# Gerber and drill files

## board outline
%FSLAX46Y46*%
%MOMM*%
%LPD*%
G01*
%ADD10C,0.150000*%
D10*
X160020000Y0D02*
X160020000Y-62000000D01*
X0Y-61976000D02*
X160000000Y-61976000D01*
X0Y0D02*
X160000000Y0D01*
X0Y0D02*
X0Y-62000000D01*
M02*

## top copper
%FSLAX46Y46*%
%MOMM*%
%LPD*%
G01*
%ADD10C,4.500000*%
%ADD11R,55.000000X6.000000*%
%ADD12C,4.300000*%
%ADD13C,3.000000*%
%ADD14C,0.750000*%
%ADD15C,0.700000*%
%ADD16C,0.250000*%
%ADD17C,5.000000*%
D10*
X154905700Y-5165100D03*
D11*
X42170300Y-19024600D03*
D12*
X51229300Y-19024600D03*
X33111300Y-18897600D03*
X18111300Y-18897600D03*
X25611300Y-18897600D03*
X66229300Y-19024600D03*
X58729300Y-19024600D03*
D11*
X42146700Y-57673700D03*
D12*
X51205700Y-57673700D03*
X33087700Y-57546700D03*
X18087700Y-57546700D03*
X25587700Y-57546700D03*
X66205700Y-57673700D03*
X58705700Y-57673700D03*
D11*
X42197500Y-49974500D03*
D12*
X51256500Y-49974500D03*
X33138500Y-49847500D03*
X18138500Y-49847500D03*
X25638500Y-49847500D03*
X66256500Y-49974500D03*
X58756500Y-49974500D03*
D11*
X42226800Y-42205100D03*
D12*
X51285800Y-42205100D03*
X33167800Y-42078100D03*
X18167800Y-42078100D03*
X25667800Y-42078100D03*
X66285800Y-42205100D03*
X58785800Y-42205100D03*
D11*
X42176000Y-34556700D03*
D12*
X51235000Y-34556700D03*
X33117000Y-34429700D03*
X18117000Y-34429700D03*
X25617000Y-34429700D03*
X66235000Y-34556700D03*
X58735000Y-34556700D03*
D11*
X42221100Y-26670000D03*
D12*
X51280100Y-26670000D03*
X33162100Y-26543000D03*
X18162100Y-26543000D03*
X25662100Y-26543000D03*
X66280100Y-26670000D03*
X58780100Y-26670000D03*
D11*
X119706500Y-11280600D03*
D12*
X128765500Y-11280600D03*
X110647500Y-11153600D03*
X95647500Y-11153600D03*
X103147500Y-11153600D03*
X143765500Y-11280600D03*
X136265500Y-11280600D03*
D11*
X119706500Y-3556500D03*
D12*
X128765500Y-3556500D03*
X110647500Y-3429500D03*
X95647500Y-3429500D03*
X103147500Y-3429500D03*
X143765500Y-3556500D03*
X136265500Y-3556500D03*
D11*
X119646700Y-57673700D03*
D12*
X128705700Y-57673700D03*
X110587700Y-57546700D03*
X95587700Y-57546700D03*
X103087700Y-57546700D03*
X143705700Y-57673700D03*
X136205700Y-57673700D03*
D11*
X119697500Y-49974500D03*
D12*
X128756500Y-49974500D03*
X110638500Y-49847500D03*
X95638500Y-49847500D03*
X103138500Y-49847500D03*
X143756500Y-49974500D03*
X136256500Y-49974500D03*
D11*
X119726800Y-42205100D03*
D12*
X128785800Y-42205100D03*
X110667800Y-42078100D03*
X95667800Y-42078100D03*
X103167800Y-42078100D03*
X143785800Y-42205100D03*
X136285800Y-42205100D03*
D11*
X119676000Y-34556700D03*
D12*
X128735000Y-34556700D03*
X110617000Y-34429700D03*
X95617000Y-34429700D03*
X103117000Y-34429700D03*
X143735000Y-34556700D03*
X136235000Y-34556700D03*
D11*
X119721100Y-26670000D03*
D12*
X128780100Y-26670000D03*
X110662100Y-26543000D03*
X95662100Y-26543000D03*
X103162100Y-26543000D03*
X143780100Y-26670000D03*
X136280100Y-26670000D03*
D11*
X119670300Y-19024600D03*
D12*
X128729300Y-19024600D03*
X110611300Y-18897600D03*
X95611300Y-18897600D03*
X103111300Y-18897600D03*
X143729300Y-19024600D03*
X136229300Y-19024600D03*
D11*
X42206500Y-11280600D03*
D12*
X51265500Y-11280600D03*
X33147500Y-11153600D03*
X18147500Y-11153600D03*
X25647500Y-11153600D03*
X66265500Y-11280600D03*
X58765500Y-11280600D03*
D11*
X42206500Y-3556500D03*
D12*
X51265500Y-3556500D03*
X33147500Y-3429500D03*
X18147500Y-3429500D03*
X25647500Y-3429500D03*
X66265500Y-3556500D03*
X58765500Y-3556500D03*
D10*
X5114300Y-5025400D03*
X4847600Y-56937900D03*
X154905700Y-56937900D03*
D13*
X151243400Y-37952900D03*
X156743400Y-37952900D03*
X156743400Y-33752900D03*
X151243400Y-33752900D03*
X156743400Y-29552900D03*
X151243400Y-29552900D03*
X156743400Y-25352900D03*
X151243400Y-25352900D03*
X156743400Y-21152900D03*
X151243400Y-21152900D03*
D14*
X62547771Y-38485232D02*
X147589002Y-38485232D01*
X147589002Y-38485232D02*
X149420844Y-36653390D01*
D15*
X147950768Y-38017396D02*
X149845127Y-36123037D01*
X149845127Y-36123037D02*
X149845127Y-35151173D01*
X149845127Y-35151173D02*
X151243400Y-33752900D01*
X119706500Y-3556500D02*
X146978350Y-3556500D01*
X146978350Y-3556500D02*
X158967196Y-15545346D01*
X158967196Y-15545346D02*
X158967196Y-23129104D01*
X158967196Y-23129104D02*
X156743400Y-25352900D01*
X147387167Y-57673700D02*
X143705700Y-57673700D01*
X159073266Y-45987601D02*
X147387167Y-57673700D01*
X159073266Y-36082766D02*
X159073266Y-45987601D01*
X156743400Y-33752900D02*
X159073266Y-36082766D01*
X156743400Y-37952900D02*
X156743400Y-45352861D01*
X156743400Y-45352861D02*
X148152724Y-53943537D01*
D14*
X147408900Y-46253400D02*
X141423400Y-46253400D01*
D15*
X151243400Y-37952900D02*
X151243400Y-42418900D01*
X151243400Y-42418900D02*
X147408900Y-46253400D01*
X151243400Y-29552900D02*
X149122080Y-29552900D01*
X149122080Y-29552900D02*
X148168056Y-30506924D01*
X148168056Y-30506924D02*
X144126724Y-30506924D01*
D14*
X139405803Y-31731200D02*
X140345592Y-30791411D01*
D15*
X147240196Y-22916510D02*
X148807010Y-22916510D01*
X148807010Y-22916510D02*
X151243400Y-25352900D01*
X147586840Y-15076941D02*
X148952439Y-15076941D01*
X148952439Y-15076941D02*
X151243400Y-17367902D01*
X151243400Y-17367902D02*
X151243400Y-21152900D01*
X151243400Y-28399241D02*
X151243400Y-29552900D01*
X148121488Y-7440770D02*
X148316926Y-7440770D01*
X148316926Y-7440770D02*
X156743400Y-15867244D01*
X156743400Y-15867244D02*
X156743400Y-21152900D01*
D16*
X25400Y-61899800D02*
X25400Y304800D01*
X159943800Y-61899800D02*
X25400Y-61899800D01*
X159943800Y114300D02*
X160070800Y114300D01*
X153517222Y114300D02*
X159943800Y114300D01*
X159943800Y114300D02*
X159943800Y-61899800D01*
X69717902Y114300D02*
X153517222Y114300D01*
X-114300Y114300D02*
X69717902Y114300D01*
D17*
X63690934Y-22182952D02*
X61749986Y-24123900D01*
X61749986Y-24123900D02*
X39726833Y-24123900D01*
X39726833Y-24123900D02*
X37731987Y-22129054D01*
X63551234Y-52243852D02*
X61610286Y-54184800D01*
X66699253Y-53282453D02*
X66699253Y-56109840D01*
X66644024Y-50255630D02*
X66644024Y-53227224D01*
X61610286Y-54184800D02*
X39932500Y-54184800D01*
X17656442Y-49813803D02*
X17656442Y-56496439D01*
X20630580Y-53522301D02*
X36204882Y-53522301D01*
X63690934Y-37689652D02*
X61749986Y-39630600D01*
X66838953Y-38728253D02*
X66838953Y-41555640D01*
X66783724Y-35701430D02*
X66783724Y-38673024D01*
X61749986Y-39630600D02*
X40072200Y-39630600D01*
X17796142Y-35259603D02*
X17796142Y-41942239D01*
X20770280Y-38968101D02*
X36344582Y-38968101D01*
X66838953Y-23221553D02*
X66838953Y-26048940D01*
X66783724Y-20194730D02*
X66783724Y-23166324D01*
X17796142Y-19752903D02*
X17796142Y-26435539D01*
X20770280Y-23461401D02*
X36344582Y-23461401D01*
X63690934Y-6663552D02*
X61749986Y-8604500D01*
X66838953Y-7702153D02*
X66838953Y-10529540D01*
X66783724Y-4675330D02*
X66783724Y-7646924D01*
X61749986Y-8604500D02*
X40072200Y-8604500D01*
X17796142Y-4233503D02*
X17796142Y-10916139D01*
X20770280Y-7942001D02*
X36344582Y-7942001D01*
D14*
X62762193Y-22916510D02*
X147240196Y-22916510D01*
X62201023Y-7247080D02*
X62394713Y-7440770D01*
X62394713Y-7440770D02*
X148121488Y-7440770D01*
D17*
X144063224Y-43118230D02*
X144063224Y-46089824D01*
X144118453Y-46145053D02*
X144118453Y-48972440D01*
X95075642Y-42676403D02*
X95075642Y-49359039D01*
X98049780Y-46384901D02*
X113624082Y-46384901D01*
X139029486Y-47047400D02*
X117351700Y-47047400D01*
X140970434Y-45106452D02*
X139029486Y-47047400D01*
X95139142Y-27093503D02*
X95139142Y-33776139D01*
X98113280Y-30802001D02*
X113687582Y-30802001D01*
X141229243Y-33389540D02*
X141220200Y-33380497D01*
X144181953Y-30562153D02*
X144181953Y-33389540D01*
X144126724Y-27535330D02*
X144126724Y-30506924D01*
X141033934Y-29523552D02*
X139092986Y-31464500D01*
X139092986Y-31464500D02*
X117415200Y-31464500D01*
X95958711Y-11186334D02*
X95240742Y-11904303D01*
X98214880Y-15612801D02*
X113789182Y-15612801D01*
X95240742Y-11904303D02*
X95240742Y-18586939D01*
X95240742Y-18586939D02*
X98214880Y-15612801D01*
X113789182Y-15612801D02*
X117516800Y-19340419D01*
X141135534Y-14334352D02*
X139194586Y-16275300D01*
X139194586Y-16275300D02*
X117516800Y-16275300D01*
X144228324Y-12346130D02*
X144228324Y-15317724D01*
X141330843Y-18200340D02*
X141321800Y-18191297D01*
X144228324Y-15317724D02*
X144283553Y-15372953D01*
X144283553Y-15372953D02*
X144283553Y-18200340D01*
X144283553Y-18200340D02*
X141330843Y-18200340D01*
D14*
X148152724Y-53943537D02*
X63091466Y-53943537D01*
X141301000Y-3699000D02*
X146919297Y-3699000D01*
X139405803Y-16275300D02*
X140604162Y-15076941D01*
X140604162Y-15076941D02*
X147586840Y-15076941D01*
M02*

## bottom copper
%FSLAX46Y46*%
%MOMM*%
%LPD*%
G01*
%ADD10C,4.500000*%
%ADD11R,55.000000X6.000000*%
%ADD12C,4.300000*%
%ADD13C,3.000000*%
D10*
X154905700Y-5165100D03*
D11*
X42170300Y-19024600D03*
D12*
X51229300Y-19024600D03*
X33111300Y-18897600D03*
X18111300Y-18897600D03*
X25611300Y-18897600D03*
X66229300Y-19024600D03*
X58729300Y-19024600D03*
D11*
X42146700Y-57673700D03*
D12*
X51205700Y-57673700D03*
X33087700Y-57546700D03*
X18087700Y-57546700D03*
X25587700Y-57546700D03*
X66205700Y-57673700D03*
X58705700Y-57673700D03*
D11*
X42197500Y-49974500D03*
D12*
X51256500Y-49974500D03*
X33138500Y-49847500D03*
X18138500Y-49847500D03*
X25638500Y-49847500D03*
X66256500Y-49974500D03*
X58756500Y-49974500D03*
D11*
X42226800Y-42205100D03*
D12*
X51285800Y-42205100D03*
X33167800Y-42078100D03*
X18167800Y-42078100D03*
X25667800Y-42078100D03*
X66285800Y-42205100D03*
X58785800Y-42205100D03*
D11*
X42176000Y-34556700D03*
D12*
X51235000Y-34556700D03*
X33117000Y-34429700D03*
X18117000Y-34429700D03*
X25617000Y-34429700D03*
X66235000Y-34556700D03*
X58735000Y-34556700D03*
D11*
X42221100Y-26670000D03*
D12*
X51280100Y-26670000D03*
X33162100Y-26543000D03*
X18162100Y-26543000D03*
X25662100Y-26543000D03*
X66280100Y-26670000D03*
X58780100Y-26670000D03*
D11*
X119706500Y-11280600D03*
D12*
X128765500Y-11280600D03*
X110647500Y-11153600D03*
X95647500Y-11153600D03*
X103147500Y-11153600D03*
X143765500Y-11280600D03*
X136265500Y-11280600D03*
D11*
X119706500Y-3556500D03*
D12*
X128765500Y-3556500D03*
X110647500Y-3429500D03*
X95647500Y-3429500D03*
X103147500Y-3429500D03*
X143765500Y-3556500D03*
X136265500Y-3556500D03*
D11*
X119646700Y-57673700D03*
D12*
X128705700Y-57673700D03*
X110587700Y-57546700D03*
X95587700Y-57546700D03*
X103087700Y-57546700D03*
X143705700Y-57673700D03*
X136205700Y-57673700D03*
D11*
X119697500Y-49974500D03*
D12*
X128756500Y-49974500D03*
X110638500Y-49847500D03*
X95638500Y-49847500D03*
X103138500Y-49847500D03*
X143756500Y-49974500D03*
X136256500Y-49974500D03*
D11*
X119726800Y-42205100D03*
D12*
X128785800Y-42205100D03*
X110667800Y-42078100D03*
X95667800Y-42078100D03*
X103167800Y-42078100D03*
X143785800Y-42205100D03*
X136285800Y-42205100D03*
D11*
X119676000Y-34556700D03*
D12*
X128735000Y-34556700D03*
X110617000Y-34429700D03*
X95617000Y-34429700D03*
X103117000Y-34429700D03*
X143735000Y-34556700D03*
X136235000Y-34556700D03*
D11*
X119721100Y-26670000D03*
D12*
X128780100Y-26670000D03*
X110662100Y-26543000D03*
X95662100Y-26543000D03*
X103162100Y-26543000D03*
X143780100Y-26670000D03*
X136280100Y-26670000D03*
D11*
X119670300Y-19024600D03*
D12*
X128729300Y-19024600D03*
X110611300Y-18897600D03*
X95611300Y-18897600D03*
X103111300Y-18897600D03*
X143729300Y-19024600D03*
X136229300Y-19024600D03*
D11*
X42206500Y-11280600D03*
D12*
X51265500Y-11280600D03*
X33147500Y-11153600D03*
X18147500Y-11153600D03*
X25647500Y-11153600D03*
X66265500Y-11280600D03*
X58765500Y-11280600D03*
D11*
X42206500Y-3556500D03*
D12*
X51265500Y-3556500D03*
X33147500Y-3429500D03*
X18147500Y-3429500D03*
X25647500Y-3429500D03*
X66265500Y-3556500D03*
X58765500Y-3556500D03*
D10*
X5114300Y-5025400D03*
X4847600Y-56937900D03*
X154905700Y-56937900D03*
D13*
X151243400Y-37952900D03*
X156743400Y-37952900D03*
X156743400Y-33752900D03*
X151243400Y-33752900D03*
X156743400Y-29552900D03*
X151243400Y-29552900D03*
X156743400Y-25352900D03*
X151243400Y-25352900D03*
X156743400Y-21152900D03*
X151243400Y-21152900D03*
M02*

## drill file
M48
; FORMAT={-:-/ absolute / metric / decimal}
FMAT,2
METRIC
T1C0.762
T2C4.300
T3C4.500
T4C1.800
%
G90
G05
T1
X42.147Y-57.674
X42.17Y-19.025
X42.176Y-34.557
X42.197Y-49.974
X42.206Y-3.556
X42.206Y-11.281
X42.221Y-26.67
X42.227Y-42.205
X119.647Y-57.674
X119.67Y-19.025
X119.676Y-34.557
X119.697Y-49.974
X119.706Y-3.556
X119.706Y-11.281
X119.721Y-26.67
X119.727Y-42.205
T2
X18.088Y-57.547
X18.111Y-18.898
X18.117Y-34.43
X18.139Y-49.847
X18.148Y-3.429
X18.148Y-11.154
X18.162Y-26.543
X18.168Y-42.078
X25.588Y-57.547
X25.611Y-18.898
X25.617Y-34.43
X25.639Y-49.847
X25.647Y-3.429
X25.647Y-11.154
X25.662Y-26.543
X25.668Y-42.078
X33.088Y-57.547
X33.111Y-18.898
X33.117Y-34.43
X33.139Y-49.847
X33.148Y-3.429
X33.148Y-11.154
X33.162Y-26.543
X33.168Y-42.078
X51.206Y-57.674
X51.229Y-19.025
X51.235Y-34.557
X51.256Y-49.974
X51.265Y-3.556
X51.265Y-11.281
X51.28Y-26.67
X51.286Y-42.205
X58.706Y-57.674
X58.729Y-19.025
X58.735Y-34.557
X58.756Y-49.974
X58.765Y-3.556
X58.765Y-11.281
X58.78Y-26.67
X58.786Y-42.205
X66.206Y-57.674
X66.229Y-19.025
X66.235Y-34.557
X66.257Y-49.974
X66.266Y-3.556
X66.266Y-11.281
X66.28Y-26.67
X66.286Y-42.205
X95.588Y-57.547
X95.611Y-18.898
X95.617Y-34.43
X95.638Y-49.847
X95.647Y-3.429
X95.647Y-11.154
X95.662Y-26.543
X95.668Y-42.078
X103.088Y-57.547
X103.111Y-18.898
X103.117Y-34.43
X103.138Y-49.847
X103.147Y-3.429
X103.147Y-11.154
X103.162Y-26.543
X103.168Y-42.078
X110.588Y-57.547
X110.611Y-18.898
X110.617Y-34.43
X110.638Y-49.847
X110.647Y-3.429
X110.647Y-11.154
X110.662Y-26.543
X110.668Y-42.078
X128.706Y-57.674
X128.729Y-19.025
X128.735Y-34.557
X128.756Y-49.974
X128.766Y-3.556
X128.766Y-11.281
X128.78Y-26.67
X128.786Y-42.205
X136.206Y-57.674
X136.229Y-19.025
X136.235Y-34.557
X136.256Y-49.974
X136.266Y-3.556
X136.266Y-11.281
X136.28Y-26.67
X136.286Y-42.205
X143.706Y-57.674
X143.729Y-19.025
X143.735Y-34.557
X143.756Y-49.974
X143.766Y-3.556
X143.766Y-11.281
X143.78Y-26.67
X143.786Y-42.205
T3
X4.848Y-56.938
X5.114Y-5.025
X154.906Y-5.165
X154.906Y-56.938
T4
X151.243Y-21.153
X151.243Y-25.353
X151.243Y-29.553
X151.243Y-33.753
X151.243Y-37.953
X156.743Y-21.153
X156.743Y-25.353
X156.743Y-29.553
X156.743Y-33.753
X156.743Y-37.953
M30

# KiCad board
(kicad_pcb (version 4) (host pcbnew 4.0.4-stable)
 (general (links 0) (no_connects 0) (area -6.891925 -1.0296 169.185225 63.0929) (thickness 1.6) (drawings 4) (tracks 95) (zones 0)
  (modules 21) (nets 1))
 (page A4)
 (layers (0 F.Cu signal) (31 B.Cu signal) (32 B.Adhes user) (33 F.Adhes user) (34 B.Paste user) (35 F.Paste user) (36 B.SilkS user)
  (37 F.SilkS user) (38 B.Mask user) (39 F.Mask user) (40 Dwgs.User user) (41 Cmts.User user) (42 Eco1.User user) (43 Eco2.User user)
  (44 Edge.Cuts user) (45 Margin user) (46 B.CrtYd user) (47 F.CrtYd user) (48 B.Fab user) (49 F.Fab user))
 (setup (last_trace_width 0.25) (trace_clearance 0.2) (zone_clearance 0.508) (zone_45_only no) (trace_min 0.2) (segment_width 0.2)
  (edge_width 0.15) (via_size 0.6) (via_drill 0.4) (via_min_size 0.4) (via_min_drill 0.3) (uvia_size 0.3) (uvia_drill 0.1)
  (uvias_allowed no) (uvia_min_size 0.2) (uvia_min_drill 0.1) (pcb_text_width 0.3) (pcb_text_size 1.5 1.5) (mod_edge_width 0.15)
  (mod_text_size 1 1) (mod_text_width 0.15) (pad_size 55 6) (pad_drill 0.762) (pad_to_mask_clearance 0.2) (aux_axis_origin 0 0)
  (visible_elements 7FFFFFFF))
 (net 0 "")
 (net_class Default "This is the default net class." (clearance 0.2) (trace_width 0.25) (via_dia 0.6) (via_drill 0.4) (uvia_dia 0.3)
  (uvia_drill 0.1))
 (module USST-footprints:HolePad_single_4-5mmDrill (layer F.Cu) (at 154.9057 5.1651)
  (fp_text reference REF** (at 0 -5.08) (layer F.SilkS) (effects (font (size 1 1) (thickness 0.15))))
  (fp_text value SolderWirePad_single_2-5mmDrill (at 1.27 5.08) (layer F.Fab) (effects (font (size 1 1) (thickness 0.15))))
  (pad "" thru_hole circle (at 0 0) (size 4.5 4.5) (drill 4.5) (layers *.Cu *.Mask)))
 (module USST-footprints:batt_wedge (layer F.Cu) (at 42.1703 19.0246)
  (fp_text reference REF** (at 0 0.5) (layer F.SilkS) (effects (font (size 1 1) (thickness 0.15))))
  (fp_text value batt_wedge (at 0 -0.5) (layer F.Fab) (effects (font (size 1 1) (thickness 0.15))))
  (pad 1 thru_hole rect (at 0 0) (size 55 6) (drill 0.762) (layers F.Cu F.Paste))
  (pad "" thru_hole circle (at 9.059 0) (size 4.3 4.3) (drill 4.3) (layers *.Cu *.Mask))
  (pad "" thru_hole circle (at -9.059 -0.127) (size 4.3 4.3) (drill 4.3) (layers *.Cu *.Mask))
  (pad "" thru_hole circle (at -24.059 -0.127) (size 4.3 4.3) (drill 4.3) (layers *.Cu *.Mask))
  (pad "" thru_hole circle (at -16.559 -0.127) (size 4.3 4.3) (drill 4.3) (layers *.Cu *.Mask))
  (pad "" thru_hole circle (at 24.059 0) (size 4.3 4.3) (drill 4.3) (layers *.Cu *.Mask))
  (pad "" thru_hole circle (at 16.559 0) (size 4.3 4.3) (drill 4.3) (layers *.Cu *.Mask)))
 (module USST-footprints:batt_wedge (layer F.Cu) (at 42.1467 57.6737)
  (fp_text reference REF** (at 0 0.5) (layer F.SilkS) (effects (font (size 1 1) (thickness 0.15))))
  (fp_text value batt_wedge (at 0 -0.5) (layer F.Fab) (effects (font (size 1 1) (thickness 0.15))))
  (pad 1 thru_hole rect (at 0 0) (size 55 6) (drill 0.762) (layers F.Cu F.Paste))
  (pad "" thru_hole circle (at 9.059 0) (size 4.3 4.3) (drill 4.3) (layers *.Cu *.Mask))
  (pad "" thru_hole circle (at -9.059 -0.127) (size 4.3 4.3) (drill 4.3) (layers *.Cu *.Mask))
  (pad "" thru_hole circle (at -24.059 -0.127) (size 4.3 4.3) (drill 4.3) (layers *.Cu *.Mask))
  (pad "" thru_hole circle (at -16.559 -0.127) (size 4.3 4.3) (drill 4.3) (layers *.Cu *.Mask))
  (pad "" thru_hole circle (at 24.059 0) (size 4.3 4.3) (drill 4.3) (layers *.Cu *.Mask))
  (pad "" thru_hole circle (at 16.559 0) (size 4.3 4.3) (drill 4.3) (layers *.Cu *.Mask)))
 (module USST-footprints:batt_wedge (layer F.Cu) (at 42.1975 49.9745)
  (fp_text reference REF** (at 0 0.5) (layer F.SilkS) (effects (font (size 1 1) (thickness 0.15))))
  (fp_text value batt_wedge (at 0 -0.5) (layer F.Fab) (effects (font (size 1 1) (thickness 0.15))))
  (pad 1 thru_hole rect (at 0 0) (size 55 6) (drill 0.762) (layers F.Cu F.Paste))
  (pad "" thru_hole circle (at 9.059 0) (size 4.3 4.3) (drill 4.3) (layers *.Cu *.Mask))
  (pad "" thru_hole circle (at -9.059 -0.127) (size 4.3 4.3) (drill 4.3) (layers *.Cu *.Mask))
  (pad "" thru_hole circle (at -24.059 -0.127) (size 4.3 4.3) (drill 4.3) (layers *.Cu *.Mask))
  (pad "" thru_hole circle (at -16.559 -0.127) (size 4.3 4.3) (drill 4.3) (layers *.Cu *.Mask))
  (pad "" thru_hole circle (at 24.059 0) (size 4.3 4.3) (drill 4.3) (layers *.Cu *.Mask))
  (pad "" thru_hole circle (at 16.559 0) (size 4.3 4.3) (drill 4.3) (layers *.Cu *.Mask)))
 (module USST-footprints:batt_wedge (layer F.Cu) (at 42.2268 42.2051)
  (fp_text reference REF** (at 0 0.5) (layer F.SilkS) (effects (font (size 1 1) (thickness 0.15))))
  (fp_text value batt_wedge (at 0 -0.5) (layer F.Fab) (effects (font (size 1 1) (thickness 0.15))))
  (pad 1 thru_hole rect (at 0 0) (size 55 6) (drill 0.762) (layers F.Cu F.Paste))
  (pad "" thru_hole circle (at 9.059 0) (size 4.3 4.3) (drill 4.3) (layers *.Cu *.Mask))
  (pad "" thru_hole circle (at -9.059 -0.127) (size 4.3 4.3) (drill 4.3) (layers *.Cu *.Mask))
  (pad "" thru_hole circle (at -24.059 -0.127) (size 4.3 4.3) (drill 4.3) (layers *.Cu *.Mask))
  (pad "" thru_hole circle (at -16.559 -0.127) (size 4.3 4.3) (drill 4.3) (layers *.Cu *.Mask))
  (pad "" thru_hole circle (at 24.059 0) (size 4.3 4.3) (drill 4.3) (layers *.Cu *.Mask))
  (pad "" thru_hole circle (at 16.559 0) (size 4.3 4.3) (drill 4.3) (layers *.Cu *.Mask)))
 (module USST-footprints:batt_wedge (layer F.Cu) (at 42.176 34.5567)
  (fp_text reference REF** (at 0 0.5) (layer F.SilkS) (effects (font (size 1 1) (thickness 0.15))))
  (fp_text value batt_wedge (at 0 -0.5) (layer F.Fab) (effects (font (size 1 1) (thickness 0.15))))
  (pad 1 thru_hole rect (at 0 0) (size 55 6) (drill 0.762) (layers F.Cu F.Paste))
  (pad "" thru_hole circle (at 9.059 0) (size 4.3 4.3) (drill 4.3) (layers *.Cu *.Mask))
  (pad "" thru_hole circle (at -9.059 -0.127) (size 4.3 4.3) (drill 4.3) (layers *.Cu *.Mask))
  (pad "" thru_hole circle (at -24.059 -0.127) (size 4.3 4.3) (drill 4.3) (layers *.Cu *.Mask))
  (pad "" thru_hole circle (at -16.559 -0.127) (size 4.3 4.3) (drill 4.3) (layers *.Cu *.Mask))
  (pad "" thru_hole circle (at 24.059 0) (size 4.3 4.3) (drill 4.3) (layers *.Cu *.Mask))
  (pad "" thru_hole circle (at 16.559 0) (size 4.3 4.3) (drill 4.3) (layers *.Cu *.Mask)))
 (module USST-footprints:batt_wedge (layer F.Cu) (at 42.2211 26.67)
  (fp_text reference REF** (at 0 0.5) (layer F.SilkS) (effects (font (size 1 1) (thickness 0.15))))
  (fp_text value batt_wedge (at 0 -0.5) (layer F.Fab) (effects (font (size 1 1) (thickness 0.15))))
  (pad 1 thru_hole rect (at 0 0) (size 55 6) (drill 0.762) (layers F.Cu F.Paste))
  (pad "" thru_hole circle (at 9.059 0) (size 4.3 4.3) (drill 4.3) (layers *.Cu *.Mask))
  (pad "" thru_hole circle (at -9.059 -0.127) (size 4.3 4.3) (drill 4.3) (layers *.Cu *.Mask))
  (pad "" thru_hole circle (at -24.059 -0.127) (size 4.3 4.3) (drill 4.3) (layers *.Cu *.Mask))
  (pad "" thru_hole circle (at -16.559 -0.127) (size 4.3 4.3) (drill 4.3) (layers *.Cu *.Mask))
  (pad "" thru_hole circle (at 24.059 0) (size 4.3 4.3) (drill 4.3) (layers *.Cu *.Mask))
  (pad "" thru_hole circle (at 16.559 0) (size 4.3 4.3) (drill 4.3) (layers *.Cu *.Mask)))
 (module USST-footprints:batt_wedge (layer F.Cu) (at 119.7065 11.2806)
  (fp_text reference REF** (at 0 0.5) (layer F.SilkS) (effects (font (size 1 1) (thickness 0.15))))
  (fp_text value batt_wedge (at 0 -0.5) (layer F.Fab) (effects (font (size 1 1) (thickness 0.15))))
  (pad 1 thru_hole rect (at 0 0) (size 55 6) (drill 0.762) (layers F.Cu F.Paste))
  (pad "" thru_hole circle (at 9.059 0) (size 4.3 4.3) (drill 4.3) (layers *.Cu *.Mask))
  (pad "" thru_hole circle (at -9.059 -0.127) (size 4.3 4.3) (drill 4.3) (layers *.Cu *.Mask))
  (pad "" thru_hole circle (at -24.059 -0.127) (size 4.3 4.3) (drill 4.3) (layers *.Cu *.Mask))
  (pad "" thru_hole circle (at -16.559 -0.127) (size 4.3 4.3) (drill 4.3) (layers *.Cu *.Mask))
  (pad "" thru_hole circle (at 24.059 0) (size 4.3 4.3) (drill 4.3) (layers *.Cu *.Mask))
  (pad "" thru_hole circle (at 16.559 0) (size 4.3 4.3) (drill 4.3) (layers *.Cu *.Mask)))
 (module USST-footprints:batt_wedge (layer F.Cu) (at 119.7065 3.5565)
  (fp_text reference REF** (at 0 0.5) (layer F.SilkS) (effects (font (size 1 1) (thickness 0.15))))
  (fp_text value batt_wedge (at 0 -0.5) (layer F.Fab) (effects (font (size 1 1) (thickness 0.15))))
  (pad 1 thru_hole rect (at 0 0) (size 55 6) (drill 0.762) (layers F.Cu F.Paste))
  (pad "" thru_hole circle (at 9.059 0) (size 4.3 4.3) (drill 4.3) (layers *.Cu *.Mask))
  (pad "" thru_hole circle (at -9.059 -0.127) (size 4.3 4.3) (drill 4.3) (layers *.Cu *.Mask))
  (pad "" thru_hole circle (at -24.059 -0.127) (size 4.3 4.3) (drill 4.3) (layers *.Cu *.Mask))
  (pad "" thru_hole circle (at -16.559 -0.127) (size 4.3 4.3) (drill 4.3) (layers *.Cu *.Mask))
  (pad "" thru_hole circle (at 24.059 0) (size 4.3 4.3) (drill 4.3) (layers *.Cu *.Mask))
  (pad "" thru_hole circle (at 16.559 0) (size 4.3 4.3) (drill 4.3) (layers *.Cu *.Mask)))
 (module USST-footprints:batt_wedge (layer F.Cu) (at 119.6467 57.6737)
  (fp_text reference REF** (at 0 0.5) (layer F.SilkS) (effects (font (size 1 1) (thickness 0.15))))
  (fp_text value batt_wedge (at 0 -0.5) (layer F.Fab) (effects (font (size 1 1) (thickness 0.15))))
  (pad 1 thru_hole rect (at 0 0) (size 55 6) (drill 0.762) (layers F.Cu F.Paste))
  (pad "" thru_hole circle (at 9.059 0) (size 4.3 4.3) (drill 4.3) (layers *.Cu *.Mask))
  (pad "" thru_hole circle (at -9.059 -0.127) (size 4.3 4.3) (drill 4.3) (layers *.Cu *.Mask))
  (pad "" thru_hole circle (at -24.059 -0.127) (size 4.3 4.3) (drill 4.3) (layers *.Cu *.Mask))
  (pad "" thru_hole circle (at -16.559 -0.127) (size 4.3 4.3) (drill 4.3) (layers *.Cu *.Mask))
  (pad "" thru_hole circle (at 24.059 0) (size 4.3 4.3) (drill 4.3) (layers *.Cu *.Mask))
  (pad "" thru_hole circle (at 16.559 0) (size 4.3 4.3) (drill 4.3) (layers *.Cu *.Mask)))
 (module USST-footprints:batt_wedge (layer F.Cu) (at 119.6975 49.9745)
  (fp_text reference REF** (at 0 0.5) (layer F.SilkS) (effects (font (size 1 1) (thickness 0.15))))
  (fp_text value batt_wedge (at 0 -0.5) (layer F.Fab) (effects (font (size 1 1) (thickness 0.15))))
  (pad 1 thru_hole rect (at 0 0) (size 55 6) (drill 0.762) (layers F.Cu F.Paste))
  (pad "" thru_hole circle (at 9.059 0) (size 4.3 4.3) (drill 4.3) (layers *.Cu *.Mask))
  (pad "" thru_hole circle (at -9.059 -0.127) (size 4.3 4.3) (drill 4.3) (layers *.Cu *.Mask))
  (pad "" thru_hole circle (at -24.059 -0.127) (size 4.3 4.3) (drill 4.3) (layers *.Cu *.Mask))
  (pad "" thru_hole circle (at -16.559 -0.127) (size 4.3 4.3) (drill 4.3) (layers *.Cu *.Mask))
  (pad "" thru_hole circle (at 24.059 0) (size 4.3 4.3) (drill 4.3) (layers *.Cu *.Mask))
  (pad "" thru_hole circle (at 16.559 0) (size 4.3 4.3) (drill 4.3) (layers *.Cu *.Mask)))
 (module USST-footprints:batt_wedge (layer F.Cu) (at 119.7268 42.2051)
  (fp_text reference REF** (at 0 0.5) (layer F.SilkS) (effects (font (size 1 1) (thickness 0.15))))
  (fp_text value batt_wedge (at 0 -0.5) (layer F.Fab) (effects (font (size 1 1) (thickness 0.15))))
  (pad 1 thru_hole rect (at 0 0) (size 55 6) (drill 0.762) (layers F.Cu F.Paste))
  (pad "" thru_hole circle (at 9.059 0) (size 4.3 4.3) (drill 4.3) (layers *.Cu *.Mask))
  (pad "" thru_hole circle (at -9.059 -0.127) (size 4.3 4.3) (drill 4.3) (layers *.Cu *.Mask))
  (pad "" thru_hole circle (at -24.059 -0.127) (size 4.3 4.3) (drill 4.3) (layers *.Cu *.Mask))
  (pad "" thru_hole circle (at -16.559 -0.127) (size 4.3 4.3) (drill 4.3) (layers *.Cu *.Mask))
  (pad "" thru_hole circle (at 24.059 0) (size 4.3 4.3) (drill 4.3) (layers *.Cu *.Mask))
  (pad "" thru_hole circle (at 16.559 0) (size 4.3 4.3) (drill 4.3) (layers *.Cu *.Mask)))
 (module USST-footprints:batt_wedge (layer F.Cu) (at 119.676 34.5567)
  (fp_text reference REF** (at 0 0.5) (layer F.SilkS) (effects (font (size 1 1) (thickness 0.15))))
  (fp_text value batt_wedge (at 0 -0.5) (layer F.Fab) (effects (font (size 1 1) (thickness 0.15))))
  (pad 1 thru_hole rect (at 0 0) (size 55 6) (drill 0.762) (layers F.Cu F.Paste))
  (pad "" thru_hole circle (at 9.059 0) (size 4.3 4.3) (drill 4.3) (layers *.Cu *.Mask))
  (pad "" thru_hole circle (at -9.059 -0.127) (size 4.3 4.3) (drill 4.3) (layers *.Cu *.Mask))
  (pad "" thru_hole circle (at -24.059 -0.127) (size 4.3 4.3) (drill 4.3) (layers *.Cu *.Mask))
  (pad "" thru_hole circle (at -16.559 -0.127) (size 4.3 4.3) (drill 4.3) (layers *.Cu *.Mask))
  (pad "" thru_hole circle (at 24.059 0) (size 4.3 4.3) (drill 4.3) (layers *.Cu *.Mask))
  (pad "" thru_hole circle (at 16.559 0) (size 4.3 4.3) (drill 4.3) (layers *.Cu *.Mask)))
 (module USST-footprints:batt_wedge (layer F.Cu) (at 119.7211 26.67)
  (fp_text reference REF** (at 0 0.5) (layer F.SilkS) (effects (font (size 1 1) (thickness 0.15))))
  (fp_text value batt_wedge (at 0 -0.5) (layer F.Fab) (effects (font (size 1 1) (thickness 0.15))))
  (pad 1 thru_hole rect (at 0 0) (size 55 6) (drill 0.762) (layers F.Cu F.Paste))
  (pad "" thru_hole circle (at 9.059 0) (size 4.3 4.3) (drill 4.3) (layers *.Cu *.Mask))
  (pad "" thru_hole circle (at -9.059 -0.127) (size 4.3 4.3) (drill 4.3) (layers *.Cu *.Mask))
  (pad "" thru_hole circle (at -24.059 -0.127) (size 4.3 4.3) (drill 4.3) (layers *.Cu *.Mask))
  (pad "" thru_hole circle (at -16.559 -0.127) (size 4.3 4.3) (drill 4.3) (layers *.Cu *.Mask))
  (pad "" thru_hole circle (at 24.059 0) (size 4.3 4.3) (drill 4.3) (layers *.Cu *.Mask))
  (pad "" thru_hole circle (at 16.559 0) (size 4.3 4.3) (drill 4.3) (layers *.Cu *.Mask)))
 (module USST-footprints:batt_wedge (layer F.Cu) (at 119.6703 19.0246)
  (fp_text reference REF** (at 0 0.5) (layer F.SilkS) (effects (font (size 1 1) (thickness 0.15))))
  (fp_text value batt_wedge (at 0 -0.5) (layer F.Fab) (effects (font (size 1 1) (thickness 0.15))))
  (pad 1 thru_hole rect (at 0 0) (size 55 6) (drill 0.762) (layers F.Cu F.Paste))
  (pad "" thru_hole circle (at 9.059 0) (size 4.3 4.3) (drill 4.3) (layers *.Cu *.Mask))
  (pad "" thru_hole circle (at -9.059 -0.127) (size 4.3 4.3) (drill 4.3) (layers *.Cu *.Mask))
  (pad "" thru_hole circle (at -24.059 -0.127) (size 4.3 4.3) (drill 4.3) (layers *.Cu *.Mask))
  (pad "" thru_hole circle (at -16.559 -0.127) (size 4.3 4.3) (drill 4.3) (layers *.Cu *.Mask))
  (pad "" thru_hole circle (at 24.059 0) (size 4.3 4.3) (drill 4.3) (layers *.Cu *.Mask))
  (pad "" thru_hole circle (at 16.559 0) (size 4.3 4.3) (drill 4.3) (layers *.Cu *.Mask)))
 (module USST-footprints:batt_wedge (layer F.Cu) (at 42.2065 11.2806)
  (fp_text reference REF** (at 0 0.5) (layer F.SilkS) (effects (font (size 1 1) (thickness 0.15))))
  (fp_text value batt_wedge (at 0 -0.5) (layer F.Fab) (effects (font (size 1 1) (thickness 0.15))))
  (pad 1 thru_hole rect (at 0 0) (size 55 6) (drill 0.762) (layers F.Cu F.Paste))
  (pad "" thru_hole circle (at 9.059 0) (size 4.3 4.3) (drill 4.3) (layers *.Cu *.Mask))
  (pad "" thru_hole circle (at -9.059 -0.127) (size 4.3 4.3) (drill 4.3) (layers *.Cu *.Mask))
  (pad "" thru_hole circle (at -24.059 -0.127) (size 4.3 4.3) (drill 4.3) (layers *.Cu *.Mask))
  (pad "" thru_hole circle (at -16.559 -0.127) (size 4.3 4.3) (drill 4.3) (layers *.Cu *.Mask))
  (pad "" thru_hole circle (at 24.059 0) (size 4.3 4.3) (drill 4.3) (layers *.Cu *.Mask))
  (pad "" thru_hole circle (at 16.559 0) (size 4.3 4.3) (drill 4.3) (layers *.Cu *.Mask)))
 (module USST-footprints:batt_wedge (layer F.Cu) (at 42.2065 3.5565)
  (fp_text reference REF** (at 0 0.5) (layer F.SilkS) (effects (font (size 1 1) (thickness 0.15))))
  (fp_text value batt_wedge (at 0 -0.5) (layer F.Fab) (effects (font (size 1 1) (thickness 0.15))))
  (pad 1 thru_hole rect (at 0 0) (size 55 6) (drill 0.762) (layers F.Cu F.Paste))
  (pad "" thru_hole circle (at 9.059 0) (size 4.3 4.3) (drill 4.3) (layers *.Cu *.Mask))
  (pad "" thru_hole circle (at -9.059 -0.127) (size 4.3 4.3) (drill 4.3) (layers *.Cu *.Mask))
  (pad "" thru_hole circle (at -24.059 -0.127) (size 4.3 4.3) (drill 4.3) (layers *.Cu *.Mask))
  (pad "" thru_hole circle (at -16.559 -0.127) (size 4.3 4.3) (drill 4.3) (layers *.Cu *.Mask))
  (pad "" thru_hole circle (at 24.059 0) (size 4.3 4.3) (drill 4.3) (layers *.Cu *.Mask))
  (pad "" thru_hole circle (at 16.559 0) (size 4.3 4.3) (drill 4.3) (layers *.Cu *.Mask)))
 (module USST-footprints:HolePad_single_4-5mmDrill (layer F.Cu) (at 5.1143 5.0254)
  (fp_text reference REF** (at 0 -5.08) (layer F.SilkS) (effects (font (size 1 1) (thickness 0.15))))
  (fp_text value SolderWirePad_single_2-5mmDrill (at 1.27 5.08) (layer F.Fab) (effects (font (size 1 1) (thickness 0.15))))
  (pad "" thru_hole circle (at 0 0) (size 4.5 4.5) (drill 4.5) (layers *.Cu *.Mask)))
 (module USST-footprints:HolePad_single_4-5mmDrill (layer F.Cu) (at 4.8476 56.9379)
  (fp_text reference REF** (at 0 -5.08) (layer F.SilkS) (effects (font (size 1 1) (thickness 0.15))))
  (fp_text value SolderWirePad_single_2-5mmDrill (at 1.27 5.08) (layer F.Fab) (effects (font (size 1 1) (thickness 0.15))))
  (pad "" thru_hole circle (at 0 0) (size 4.5 4.5) (drill 4.5) (layers *.Cu *.Mask)))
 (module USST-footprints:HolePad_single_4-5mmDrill (layer F.Cu) (at 154.9057 56.9379)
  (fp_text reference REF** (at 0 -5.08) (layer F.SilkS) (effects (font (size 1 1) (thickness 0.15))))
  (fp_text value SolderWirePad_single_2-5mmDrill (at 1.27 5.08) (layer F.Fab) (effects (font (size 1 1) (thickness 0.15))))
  (pad "" thru_hole circle (at 0 0) (size 4.5 4.5) (drill 4.5) (layers *.Cu *.Mask)))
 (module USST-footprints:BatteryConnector (layer F.Cu) (at 151.2434 37.9529)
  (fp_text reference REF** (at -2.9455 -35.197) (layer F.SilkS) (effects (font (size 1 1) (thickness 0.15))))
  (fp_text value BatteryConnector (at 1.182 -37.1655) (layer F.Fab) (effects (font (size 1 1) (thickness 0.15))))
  (pad "" np_thru_hole circle (at 0 0) (size 3 3) (drill 1.8) (layers *.Cu))
  (pad "" np_thru_hole circle (at 5.5 0) (size 3 3) (drill 1.8) (layers *.Cu))
  (pad "" np_thru_hole circle (at 5.5 -4.2) (size 3 3) (drill 1.8) (layers *.Cu))
  (pad "" np_thru_hole circle (at 0 -4.2) (size 3 3) (drill 1.8) (layers *.Cu))
  (pad "" np_thru_hole circle (at 5.5 -8.4) (size 3 3) (drill 1.8) (layers *.Cu))
  (pad "" np_thru_hole circle (at 0 -8.4) (size 3 3) (drill 1.8) (layers *.Cu))
  (pad "" np_thru_hole circle (at 5.5 -12.6) (size 3 3) (drill 1.8) (layers *.Cu))
  (pad "" np_thru_hole circle (at 0 -12.6) (size 3 3) (drill 1.8) (layers *.Cu))
  (pad "" np_thru_hole circle (at 5.5 -16.8) (size 3 3) (drill 1.8) (layers *.Cu))
  (pad "" np_thru_hole circle (at 0 -16.8) (size 3 3) (drill 1.8) (layers *.Cu)))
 (gr_line (start 160.02 0) (end 160.02 62) (layer Edge.Cuts) (width 0.15))
 (gr_line (start 0 61.976) (end 160 61.976) (layer Edge.Cuts) (width 0.15))
 (gr_line (start 0 0) (end 160 0) (layer Edge.Cuts) (width 0.15))
 (gr_line (start 0 0) (end 0 62) (layer Edge.Cuts) (width 0.15))
 (segment (start 62.547771 38.485232) (end 147.589002 38.485232) (width 0.75) (layer F.Cu) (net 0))
 (segment (start 147.589002 38.485232) (end 149.420844 36.65339) (width 0.75) (layer F.Cu) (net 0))
 (segment (start 147.950768 38.017396) (end 149.845127 36.123037) (width 0.7) (layer F.Cu) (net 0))
 (segment (start 149.845127 36.123037) (end 149.845127 35.151173) (width 0.7) (layer F.Cu) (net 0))
 (segment (start 149.845127 35.151173) (end 151.2434 33.7529) (width 0.7) (layer F.Cu) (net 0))
 (segment (start 119.7065 3.5565) (end 146.97835 3.5565) (width 0.7) (layer F.Cu) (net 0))
 (segment (start 146.97835 3.5565) (end 158.967196 15.545346) (width 0.7) (layer F.Cu) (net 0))
 (segment (start 158.967196 15.545346) (end 158.967196 23.129104) (width 0.7) (layer F.Cu) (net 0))
 (segment (start 158.967196 23.129104) (end 156.7434 25.3529) (width 0.7) (layer F.Cu) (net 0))
 (segment (start 147.387167 57.6737) (end 143.7057 57.6737) (width 0.7) (layer F.Cu) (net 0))
 (segment (start 159.073266 45.987601) (end 147.387167 57.6737) (width 0.7) (layer F.Cu) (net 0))
 (segment (start 159.073266 36.082766) (end 159.073266 45.987601) (width 0.7) (layer F.Cu) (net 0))
 (segment (start 156.7434 33.7529) (end 159.073266 36.082766) (width 0.7) (layer F.Cu) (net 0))
 (segment (start 156.7434 37.9529) (end 156.7434 45.352861) (width 0.7) (layer F.Cu) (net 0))
 (segment (start 156.7434 45.352861) (end 148.152724 53.943537) (width 0.7) (layer F.Cu) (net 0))
 (segment (start 147.4089 46.2534) (end 141.4234 46.2534) (width 0.75) (layer F.Cu) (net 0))
 (segment (start 151.2434 37.9529) (end 151.2434 42.4189) (width 0.7) (layer F.Cu) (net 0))
 (segment (start 151.2434 42.4189) (end 147.4089 46.2534) (width 0.7) (layer F.Cu) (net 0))
 (segment (start 151.2434 29.5529) (end 149.12208 29.5529) (width 0.7) (layer F.Cu) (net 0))
 (segment (start 149.12208 29.5529) (end 148.168056 30.506924) (width 0.7) (layer F.Cu) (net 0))
 (segment (start 148.168056 30.506924) (end 144.126724 30.506924) (width 0.7) (layer F.Cu) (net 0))
 (segment (start 139.405803 31.7312) (end 140.345592 30.791411) (width 0.75) (layer F.Cu) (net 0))
 (segment (start 147.240196 22.91651) (end 148.80701 22.91651) (width 0.7) (layer F.Cu) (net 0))
 (segment (start 148.80701 22.91651) (end 151.2434 25.3529) (width 0.7) (layer F.Cu) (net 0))
 (segment (start 147.58684 15.076941) (end 148.952439 15.076941) (width 0.7) (layer F.Cu) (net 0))
 (segment (start 148.952439 15.076941) (end 151.2434 17.367902) (width 0.7) (layer F.Cu) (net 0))
 (segment (start 151.2434 17.367902) (end 151.2434 21.1529) (width 0.7) (layer F.Cu) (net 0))
 (segment (start 151.2434 28.399241) (end 151.2434 29.5529) (width 0.7) (layer F.Cu) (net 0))
 (segment (start 148.121488 7.44077) (end 148.316926 7.44077) (width 0.7) (layer F.Cu) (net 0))
 (segment (start 148.316926 7.44077) (end 156.7434 15.867244) (width 0.7) (layer F.Cu) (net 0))
 (segment (start 156.7434 15.867244) (end 156.7434 21.1529) (width 0.7) (layer F.Cu) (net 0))
 (segment (start 0.0254 61.8998) (end 0.0254 -0.3048) (width 0.25) (layer F.Cu) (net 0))
 (segment (start 159.9438 61.8998) (end 0.0254 61.8998) (width 0.25) (layer F.Cu) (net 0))
 (segment (start 159.9438 -0.1143) (end 160.0708 -0.1143) (width 0.25) (layer F.Cu) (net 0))
 (segment (start 153.517222 -0.1143) (end 159.9438 -0.1143) (width 0.25) (layer F.Cu) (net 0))
 (segment (start 159.9438 -0.1143) (end 159.9438 61.8998) (width 0.25) (layer F.Cu) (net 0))
 (segment (start 69.717902 -0.1143) (end 153.517222 -0.1143) (width 0.25) (layer F.Cu) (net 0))
 (segment (start -0.1143 -0.1143) (end 69.717902 -0.1143) (width 0.25) (layer F.Cu) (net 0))
 (segment (start 63.690934 22.182952) (end 61.749986 24.1239) (width 5) (layer F.Cu) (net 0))
 (segment (start 61.749986 24.1239) (end 39.726833 24.1239) (width 5) (layer F.Cu) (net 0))
 (segment (start 39.726833 24.1239) (end 37.731987 22.129054) (width 5) (layer F.Cu) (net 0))
 (segment (start 63.551234 52.243852) (end 61.610286 54.1848) (width 5) (layer F.Cu) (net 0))
 (segment (start 66.699253 53.282453) (end 66.699253 56.10984) (width 5) (layer F.Cu) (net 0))
 (segment (start 66.644024 50.25563) (end 66.644024 53.227224) (width 5) (layer F.Cu) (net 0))
 (segment (start 61.610286 54.1848) (end 39.9325 54.1848) (width 5) (layer F.Cu) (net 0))
 (segment (start 17.656442 49.813803) (end 17.656442 56.496439) (width 5) (layer F.Cu) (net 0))
 (segment (start 20.63058 53.522301) (end 36.204882 53.522301) (width 5) (layer F.Cu) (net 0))
 (segment (start 63.690934 37.689652) (end 61.749986 39.6306) (width 5) (layer F.Cu) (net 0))
 (segment (start 66.838953 38.728253) (end 66.838953 41.55564) (width 5) (layer F.Cu) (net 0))
 (segment (start 66.783724 35.70143) (end 66.783724 38.673024) (width 5) (layer F.Cu) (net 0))
 (segment (start 61.749986 39.6306) (end 40.0722 39.6306) (width 5) (layer F.Cu) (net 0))
 (segment (start 17.796142 35.259603) (end 17.796142 41.942239) (width 5) (layer F.Cu) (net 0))
 (segment (start 20.77028 38.968101) (end 36.344582 38.968101) (width 5) (layer F.Cu) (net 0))
 (segment (start 66.838953 23.221553) (end 66.838953 26.04894) (width 5) (layer F.Cu) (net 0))
 (segment (start 66.783724 20.19473) (end 66.783724 23.166324) (width 5) (layer F.Cu) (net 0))
 (segment (start 17.796142 19.752903) (end 17.796142 26.435539) (width 5) (layer F.Cu) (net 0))
 (segment (start 20.77028 23.461401) (end 36.344582 23.461401) (width 5) (layer F.Cu) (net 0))
 (segment (start 63.690934 6.663552) (end 61.749986 8.6045) (width 5) (layer F.Cu) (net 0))
 (segment (start 66.838953 7.702153) (end 66.838953 10.52954) (width 5) (layer F.Cu) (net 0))
 (segment (start 66.783724 4.67533) (end 66.783724 7.646924) (width 5) (layer F.Cu) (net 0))
 (segment (start 61.749986 8.6045) (end 40.0722 8.6045) (width 5) (layer F.Cu) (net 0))
 (segment (start 17.796142 4.233503) (end 17.796142 10.916139) (width 5) (layer F.Cu) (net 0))
 (segment (start 20.77028 7.942001) (end 36.344582 7.942001) (width 5) (layer F.Cu) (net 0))
 (segment (start 62.762193 22.91651) (end 147.240196 22.91651) (width 0.75) (layer F.Cu) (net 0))
 (segment (start 62.201023 7.24708) (end 62.394713 7.44077) (width 0.75) (layer F.Cu) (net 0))
 (segment (start 62.394713 7.44077) (end 148.121488 7.44077) (width 0.75) (layer F.Cu) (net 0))
 (segment (start 144.063224 43.11823) (end 144.063224 46.089824) (width 5) (layer F.Cu) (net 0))
 (segment (start 144.118453 46.145053) (end 144.118453 48.97244) (width 5) (layer F.Cu) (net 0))
 (segment (start 95.075642 42.676403) (end 95.075642 49.359039) (width 5) (layer F.Cu) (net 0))
 (segment (start 98.04978 46.384901) (end 113.624082 46.384901) (width 5) (layer F.Cu) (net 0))
 (segment (start 139.029486 47.0474) (end 117.3517 47.0474) (width 5) (layer F.Cu) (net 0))
 (segment (start 140.970434 45.106452) (end 139.029486 47.0474) (width 5) (layer F.Cu) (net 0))
 (segment (start 95.139142 27.093503) (end 95.139142 33.776139) (width 5) (layer F.Cu) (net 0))
 (segment (start 98.11328 30.802001) (end 113.687582 30.802001) (width 5) (layer F.Cu) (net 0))
 (segment (start 141.229243 33.38954) (end 141.2202 33.380497) (width 5) (layer F.Cu) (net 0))
 (segment (start 144.181953 30.562153) (end 144.181953 33.38954) (width 5) (layer F.Cu) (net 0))
 (segment (start 144.126724 27.53533) (end 144.126724 30.506924) (width 5) (layer F.Cu) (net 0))
 (segment (start 141.033934 29.523552) (end 139.092986 31.4645) (width 5) (layer F.Cu) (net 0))
 (segment (start 139.092986 31.4645) (end 117.4152 31.4645) (width 5) (layer F.Cu) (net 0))
 (segment (start 95.958711 11.186334) (end 95.240742 11.904303) (width 5) (layer F.Cu) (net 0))
 (segment (start 98.21488 15.612801) (end 113.789182 15.612801) (width 5) (layer F.Cu) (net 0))
 (segment (start 95.240742 11.904303) (end 95.240742 18.586939) (width 5) (layer F.Cu) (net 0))
 (segment (start 95.240742 18.586939) (end 98.21488 15.612801) (width 5) (layer F.Cu) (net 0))
 (segment (start 113.789182 15.612801) (end 117.5168 19.340419) (width 5) (layer F.Cu) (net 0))
 (segment (start 141.135534 14.334352) (end 139.194586 16.2753) (width 5) (layer F.Cu) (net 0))
 (segment (start 139.194586 16.2753) (end 117.5168 16.2753) (width 5) (layer F.Cu) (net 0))
 (segment (start 144.228324 12.34613) (end 144.228324 15.317724) (width 5) (layer F.Cu) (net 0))
 (segment (start 141.330843 18.20034) (end 141.3218 18.191297) (width 5) (layer F.Cu) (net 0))
 (segment (start 144.228324 15.317724) (end 144.283553 15.372953) (width 5) (layer F.Cu) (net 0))
 (segment (start 144.283553 15.372953) (end 144.283553 18.20034) (width 5) (layer F.Cu) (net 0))
 (segment (start 144.283553 18.20034) (end 141.330843 18.20034) (width 5) (layer F.Cu) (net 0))
 (segment (start 148.152724 53.943537) (end 63.091466 53.943537) (width 0.75) (layer F.Cu) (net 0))
 (segment (start 141.301 3.699) (end 146.919297 3.699) (width 0.75) (layer F.Cu) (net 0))
 (segment (start 139.405803 16.2753) (end 140.604162 15.076941) (width 0.75) (layer F.Cu) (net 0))
 (segment (start 140.604162 15.076941) (end 147.58684 15.076941) (width 0.75) (layer F.Cu) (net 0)))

